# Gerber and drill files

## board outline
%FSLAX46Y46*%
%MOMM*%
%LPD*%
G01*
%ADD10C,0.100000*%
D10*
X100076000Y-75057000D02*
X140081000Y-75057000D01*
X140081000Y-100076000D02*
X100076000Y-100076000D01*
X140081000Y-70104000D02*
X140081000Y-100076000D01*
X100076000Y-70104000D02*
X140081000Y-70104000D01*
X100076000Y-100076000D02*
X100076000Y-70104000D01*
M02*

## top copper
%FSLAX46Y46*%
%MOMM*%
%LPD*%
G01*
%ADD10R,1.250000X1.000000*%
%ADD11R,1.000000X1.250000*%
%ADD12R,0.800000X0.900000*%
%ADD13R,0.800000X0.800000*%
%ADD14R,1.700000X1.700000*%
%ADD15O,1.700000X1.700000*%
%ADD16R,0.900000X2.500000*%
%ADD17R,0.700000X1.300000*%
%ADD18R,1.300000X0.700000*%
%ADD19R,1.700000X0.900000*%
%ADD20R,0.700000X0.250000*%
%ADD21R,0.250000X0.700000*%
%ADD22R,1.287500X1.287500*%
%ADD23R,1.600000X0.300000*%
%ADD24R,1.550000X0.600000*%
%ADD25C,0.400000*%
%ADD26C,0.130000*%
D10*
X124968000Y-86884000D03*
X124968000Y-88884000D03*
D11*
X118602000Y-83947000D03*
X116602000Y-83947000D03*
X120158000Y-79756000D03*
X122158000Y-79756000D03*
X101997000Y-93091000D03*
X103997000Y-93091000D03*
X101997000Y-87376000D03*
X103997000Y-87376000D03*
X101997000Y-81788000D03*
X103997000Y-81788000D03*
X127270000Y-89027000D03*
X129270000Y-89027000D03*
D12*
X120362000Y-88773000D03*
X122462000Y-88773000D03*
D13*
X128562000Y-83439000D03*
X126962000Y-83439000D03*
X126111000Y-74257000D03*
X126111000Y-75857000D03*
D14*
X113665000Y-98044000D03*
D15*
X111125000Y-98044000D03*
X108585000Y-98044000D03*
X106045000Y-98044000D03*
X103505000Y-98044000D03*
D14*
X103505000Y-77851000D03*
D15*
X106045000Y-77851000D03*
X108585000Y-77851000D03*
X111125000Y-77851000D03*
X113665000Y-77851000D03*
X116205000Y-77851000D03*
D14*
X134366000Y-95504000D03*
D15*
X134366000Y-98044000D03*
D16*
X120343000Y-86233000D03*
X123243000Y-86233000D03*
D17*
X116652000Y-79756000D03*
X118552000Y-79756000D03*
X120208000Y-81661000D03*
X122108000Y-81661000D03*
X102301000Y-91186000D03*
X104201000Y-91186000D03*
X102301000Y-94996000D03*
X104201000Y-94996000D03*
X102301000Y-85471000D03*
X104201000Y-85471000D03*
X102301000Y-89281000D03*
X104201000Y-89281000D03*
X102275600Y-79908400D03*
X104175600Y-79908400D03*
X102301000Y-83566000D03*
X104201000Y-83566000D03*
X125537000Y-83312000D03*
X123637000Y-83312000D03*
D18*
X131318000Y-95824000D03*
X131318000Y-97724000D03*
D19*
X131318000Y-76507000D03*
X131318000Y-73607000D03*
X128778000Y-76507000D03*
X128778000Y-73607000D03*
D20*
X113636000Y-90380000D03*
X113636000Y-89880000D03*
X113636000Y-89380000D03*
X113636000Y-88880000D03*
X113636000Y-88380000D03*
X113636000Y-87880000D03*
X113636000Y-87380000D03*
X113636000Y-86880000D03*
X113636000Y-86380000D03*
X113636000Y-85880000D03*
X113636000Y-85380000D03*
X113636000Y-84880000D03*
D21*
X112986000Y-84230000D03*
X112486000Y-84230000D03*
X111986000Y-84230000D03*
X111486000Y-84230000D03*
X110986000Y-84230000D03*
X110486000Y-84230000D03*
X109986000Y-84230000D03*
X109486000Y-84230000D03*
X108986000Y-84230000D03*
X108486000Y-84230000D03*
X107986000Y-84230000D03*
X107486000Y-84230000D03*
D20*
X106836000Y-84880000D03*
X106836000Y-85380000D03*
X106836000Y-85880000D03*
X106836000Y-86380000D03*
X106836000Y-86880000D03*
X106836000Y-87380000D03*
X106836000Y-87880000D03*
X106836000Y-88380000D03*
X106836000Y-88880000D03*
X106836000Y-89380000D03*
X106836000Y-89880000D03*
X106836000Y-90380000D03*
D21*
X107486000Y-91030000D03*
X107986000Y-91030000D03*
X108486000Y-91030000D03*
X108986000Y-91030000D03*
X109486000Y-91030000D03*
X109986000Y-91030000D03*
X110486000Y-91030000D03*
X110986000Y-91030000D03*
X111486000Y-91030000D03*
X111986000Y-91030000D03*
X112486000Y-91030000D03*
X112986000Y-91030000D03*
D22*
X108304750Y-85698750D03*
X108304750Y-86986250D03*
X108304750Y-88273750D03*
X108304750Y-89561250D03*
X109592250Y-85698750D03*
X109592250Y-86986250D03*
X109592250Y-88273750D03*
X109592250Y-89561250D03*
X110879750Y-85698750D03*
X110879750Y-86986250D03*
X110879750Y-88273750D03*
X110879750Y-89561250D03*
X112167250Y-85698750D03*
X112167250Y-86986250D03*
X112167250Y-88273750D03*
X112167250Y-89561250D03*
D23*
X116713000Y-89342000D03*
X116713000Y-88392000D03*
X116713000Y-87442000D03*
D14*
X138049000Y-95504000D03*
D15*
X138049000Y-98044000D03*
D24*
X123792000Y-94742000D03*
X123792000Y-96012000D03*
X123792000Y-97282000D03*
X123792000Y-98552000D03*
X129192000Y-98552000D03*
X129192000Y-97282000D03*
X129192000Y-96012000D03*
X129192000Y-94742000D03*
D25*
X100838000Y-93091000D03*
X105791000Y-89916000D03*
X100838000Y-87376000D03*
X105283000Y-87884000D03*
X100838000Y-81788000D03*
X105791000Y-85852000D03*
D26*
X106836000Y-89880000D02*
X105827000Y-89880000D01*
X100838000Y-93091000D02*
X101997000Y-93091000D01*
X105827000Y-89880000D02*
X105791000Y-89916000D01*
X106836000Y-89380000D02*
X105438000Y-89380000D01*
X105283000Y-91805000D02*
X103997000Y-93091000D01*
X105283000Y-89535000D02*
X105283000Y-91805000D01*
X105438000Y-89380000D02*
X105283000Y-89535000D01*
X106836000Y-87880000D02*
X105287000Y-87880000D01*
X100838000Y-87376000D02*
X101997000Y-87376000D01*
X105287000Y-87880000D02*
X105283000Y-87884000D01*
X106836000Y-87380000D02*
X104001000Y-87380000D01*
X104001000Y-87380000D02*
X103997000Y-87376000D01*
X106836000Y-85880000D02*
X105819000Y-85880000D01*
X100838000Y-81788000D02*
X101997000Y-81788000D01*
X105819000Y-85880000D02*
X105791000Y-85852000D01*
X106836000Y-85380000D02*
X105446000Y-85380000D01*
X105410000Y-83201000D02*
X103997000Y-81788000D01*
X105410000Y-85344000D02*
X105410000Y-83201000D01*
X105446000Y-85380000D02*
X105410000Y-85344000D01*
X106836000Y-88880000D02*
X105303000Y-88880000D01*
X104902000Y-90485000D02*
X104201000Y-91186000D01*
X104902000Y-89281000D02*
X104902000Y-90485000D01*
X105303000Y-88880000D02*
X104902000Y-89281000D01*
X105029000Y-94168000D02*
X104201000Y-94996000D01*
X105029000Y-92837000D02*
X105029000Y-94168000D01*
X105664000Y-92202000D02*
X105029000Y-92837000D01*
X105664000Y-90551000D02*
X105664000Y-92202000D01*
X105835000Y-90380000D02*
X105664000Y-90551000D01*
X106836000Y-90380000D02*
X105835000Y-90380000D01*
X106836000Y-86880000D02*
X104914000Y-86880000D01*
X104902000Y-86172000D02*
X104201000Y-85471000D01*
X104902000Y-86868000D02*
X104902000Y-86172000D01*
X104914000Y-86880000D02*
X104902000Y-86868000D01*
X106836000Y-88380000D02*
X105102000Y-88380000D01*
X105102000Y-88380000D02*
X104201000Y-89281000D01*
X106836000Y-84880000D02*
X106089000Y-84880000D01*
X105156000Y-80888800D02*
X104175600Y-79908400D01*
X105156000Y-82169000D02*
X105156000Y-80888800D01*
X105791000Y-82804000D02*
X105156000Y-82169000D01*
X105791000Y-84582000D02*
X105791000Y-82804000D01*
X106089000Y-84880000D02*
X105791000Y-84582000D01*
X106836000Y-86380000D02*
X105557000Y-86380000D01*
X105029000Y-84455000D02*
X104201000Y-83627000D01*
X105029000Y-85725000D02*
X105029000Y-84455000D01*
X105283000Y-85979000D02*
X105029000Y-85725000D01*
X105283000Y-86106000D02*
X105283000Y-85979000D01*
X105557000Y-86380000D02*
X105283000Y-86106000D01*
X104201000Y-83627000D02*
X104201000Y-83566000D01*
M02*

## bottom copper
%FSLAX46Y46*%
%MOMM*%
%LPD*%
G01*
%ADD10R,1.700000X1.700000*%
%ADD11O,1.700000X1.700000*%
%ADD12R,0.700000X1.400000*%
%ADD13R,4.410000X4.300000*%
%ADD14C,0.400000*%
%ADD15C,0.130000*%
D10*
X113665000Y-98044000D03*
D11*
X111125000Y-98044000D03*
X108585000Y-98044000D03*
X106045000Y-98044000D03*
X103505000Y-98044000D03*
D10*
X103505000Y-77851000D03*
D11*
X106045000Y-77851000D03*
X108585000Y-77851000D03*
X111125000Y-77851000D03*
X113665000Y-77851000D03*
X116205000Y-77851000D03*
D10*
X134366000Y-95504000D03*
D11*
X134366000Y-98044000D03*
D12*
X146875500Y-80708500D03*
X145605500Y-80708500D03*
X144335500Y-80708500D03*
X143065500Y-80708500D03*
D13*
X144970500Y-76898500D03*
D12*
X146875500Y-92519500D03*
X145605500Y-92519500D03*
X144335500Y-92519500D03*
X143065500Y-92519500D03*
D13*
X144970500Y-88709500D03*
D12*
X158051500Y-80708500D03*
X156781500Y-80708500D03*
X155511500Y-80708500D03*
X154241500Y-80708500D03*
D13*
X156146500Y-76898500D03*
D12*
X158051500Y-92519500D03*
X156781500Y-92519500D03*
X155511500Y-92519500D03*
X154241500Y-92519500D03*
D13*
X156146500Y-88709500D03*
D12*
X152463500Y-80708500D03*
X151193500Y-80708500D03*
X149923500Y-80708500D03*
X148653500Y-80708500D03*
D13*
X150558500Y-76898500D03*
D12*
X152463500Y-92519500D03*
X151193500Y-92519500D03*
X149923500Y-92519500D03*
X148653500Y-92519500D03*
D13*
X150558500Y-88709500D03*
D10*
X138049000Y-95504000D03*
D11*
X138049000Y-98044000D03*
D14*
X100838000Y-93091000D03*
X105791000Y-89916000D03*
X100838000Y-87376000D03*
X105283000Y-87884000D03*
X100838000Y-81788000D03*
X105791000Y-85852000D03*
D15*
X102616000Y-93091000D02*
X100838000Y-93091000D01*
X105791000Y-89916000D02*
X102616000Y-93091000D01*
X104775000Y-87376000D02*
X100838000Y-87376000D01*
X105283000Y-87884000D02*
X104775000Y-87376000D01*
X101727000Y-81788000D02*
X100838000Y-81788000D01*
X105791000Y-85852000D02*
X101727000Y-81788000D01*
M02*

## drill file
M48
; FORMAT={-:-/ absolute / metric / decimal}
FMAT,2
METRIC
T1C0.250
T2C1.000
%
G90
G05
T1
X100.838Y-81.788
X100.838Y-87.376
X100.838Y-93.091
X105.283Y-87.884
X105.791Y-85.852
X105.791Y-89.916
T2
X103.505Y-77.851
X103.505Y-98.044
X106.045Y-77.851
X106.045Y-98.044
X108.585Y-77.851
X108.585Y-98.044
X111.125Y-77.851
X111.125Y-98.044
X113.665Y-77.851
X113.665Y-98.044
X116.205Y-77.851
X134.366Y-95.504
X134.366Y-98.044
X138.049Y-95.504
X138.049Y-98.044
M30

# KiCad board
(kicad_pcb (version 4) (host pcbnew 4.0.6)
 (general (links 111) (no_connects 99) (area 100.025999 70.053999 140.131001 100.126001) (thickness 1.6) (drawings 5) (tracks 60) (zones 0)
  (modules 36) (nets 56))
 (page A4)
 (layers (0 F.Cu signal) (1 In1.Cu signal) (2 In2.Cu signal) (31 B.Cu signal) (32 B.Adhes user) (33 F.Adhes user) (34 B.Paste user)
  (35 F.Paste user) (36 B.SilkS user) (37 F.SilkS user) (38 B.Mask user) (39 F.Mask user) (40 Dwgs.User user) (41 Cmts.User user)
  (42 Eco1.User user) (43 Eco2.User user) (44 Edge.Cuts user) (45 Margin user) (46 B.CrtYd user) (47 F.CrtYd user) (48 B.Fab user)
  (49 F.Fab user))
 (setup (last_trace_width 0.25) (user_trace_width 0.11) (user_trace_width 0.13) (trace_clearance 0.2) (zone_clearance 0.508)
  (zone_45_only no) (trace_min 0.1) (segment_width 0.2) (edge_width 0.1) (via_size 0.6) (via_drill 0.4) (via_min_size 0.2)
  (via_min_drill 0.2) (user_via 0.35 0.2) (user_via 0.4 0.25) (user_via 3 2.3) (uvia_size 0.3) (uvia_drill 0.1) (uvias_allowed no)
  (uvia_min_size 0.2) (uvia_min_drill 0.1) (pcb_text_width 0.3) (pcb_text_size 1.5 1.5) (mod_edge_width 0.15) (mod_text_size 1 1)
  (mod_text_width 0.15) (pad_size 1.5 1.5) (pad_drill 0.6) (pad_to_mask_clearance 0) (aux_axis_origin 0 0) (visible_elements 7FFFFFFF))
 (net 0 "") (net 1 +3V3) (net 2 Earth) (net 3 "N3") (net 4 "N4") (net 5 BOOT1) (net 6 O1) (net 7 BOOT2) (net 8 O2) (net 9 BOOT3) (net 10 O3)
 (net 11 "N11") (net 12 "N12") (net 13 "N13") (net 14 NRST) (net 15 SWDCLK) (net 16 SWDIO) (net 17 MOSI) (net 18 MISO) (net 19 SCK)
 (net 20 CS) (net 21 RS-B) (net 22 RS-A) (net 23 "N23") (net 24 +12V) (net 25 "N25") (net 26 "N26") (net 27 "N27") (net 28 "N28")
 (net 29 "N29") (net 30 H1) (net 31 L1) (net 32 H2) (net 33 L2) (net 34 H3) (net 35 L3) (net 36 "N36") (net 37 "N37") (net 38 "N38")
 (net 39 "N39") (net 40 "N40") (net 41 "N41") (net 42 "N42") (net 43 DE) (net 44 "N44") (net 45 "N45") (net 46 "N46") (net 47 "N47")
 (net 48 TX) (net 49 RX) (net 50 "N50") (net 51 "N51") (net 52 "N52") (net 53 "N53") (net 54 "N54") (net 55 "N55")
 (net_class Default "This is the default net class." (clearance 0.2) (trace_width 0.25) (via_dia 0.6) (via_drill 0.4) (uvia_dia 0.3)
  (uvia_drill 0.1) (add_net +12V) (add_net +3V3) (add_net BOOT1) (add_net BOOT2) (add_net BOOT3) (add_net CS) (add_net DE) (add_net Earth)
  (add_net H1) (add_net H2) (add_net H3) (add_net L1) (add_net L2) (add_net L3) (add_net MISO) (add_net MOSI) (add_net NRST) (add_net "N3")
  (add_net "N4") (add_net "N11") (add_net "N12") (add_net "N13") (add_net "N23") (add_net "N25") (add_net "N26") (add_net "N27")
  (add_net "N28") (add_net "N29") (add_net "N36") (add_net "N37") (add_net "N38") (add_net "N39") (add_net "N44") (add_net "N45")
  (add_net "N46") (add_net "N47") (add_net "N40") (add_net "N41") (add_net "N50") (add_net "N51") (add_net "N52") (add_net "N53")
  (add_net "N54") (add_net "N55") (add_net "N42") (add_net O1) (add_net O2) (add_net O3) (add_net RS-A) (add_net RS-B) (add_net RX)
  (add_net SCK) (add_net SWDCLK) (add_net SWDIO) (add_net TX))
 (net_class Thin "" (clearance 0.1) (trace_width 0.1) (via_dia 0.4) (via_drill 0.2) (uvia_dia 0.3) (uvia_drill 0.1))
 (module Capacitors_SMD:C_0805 (layer F.Cu) (at 124.968 87.884 270)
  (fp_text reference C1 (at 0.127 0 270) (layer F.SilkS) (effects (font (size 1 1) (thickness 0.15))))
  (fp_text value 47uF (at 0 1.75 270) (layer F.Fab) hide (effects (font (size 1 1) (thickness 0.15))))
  (pad 1 smd rect (at -1 0 270) (size 1 1.25) (layers F.Cu F.Paste F.Mask) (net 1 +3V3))
  (pad 2 smd rect (at 1 0 270) (size 1 1.25) (layers F.Cu F.Paste F.Mask) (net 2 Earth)))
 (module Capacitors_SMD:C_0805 (layer F.Cu) (at 117.602 83.947 180)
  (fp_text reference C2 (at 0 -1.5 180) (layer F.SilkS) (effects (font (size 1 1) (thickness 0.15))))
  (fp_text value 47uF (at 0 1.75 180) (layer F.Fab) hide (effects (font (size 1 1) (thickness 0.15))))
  (pad 1 smd rect (at -1 0 180) (size 1 1.25) (layers F.Cu F.Paste F.Mask) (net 2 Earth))
  (pad 2 smd rect (at 1 0 180) (size 1 1.25) (layers F.Cu F.Paste F.Mask) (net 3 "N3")))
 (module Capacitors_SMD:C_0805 (layer F.Cu) (at 121.158 79.756)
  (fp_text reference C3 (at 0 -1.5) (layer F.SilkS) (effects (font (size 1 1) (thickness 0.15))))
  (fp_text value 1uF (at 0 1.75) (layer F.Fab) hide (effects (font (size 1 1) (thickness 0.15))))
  (pad 1 smd rect (at -1 0) (size 1 1.25) (layers F.Cu F.Paste F.Mask) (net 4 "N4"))
  (pad 2 smd rect (at 1 0) (size 1 1.25) (layers F.Cu F.Paste F.Mask) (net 2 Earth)))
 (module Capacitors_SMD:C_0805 (layer F.Cu) (at 102.997 93.091)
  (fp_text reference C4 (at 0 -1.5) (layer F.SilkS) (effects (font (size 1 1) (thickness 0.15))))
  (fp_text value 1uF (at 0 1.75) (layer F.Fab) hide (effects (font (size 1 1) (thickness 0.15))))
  (pad 1 smd rect (at -1 0) (size 1 1.25) (layers F.Cu F.Paste F.Mask) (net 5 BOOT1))
  (pad 2 smd rect (at 1 0) (size 1 1.25) (layers F.Cu F.Paste F.Mask) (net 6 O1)))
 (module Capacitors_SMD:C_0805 (layer F.Cu) (at 102.997 87.376)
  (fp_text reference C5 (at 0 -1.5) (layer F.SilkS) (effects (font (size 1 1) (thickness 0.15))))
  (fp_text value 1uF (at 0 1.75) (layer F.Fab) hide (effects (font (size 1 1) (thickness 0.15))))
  (pad 1 smd rect (at -1 0) (size 1 1.25) (layers F.Cu F.Paste F.Mask) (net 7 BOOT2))
  (pad 2 smd rect (at 1 0) (size 1 1.25) (layers F.Cu F.Paste F.Mask) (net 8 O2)))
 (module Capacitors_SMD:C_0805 (layer F.Cu) (at 102.997 81.788)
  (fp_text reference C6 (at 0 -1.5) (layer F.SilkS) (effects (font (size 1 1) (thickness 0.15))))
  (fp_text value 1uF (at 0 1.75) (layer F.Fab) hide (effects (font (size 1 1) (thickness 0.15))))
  (pad 1 smd rect (at -1 0) (size 1 1.25) (layers F.Cu F.Paste F.Mask) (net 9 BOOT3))
  (pad 2 smd rect (at 1 0) (size 1 1.25) (layers F.Cu F.Paste F.Mask) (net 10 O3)))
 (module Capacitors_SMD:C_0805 (layer F.Cu) (at 128.27 89.027)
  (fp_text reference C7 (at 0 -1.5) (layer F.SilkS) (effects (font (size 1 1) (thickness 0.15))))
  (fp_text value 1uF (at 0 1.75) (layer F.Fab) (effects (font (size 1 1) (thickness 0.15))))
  (pad 1 smd rect (at -1 0) (size 1 1.25) (layers F.Cu F.Paste F.Mask) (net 2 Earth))
  (pad 2 smd rect (at 1 0) (size 1 1.25) (layers F.Cu F.Paste F.Mask) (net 1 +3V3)))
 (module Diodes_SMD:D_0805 (layer F.Cu) (at 121.412 88.773)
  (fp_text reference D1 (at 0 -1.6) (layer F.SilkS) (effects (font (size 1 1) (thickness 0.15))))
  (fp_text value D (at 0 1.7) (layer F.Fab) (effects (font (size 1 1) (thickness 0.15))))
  (pad 1 smd rect (at -1.05 0) (size 0.8 0.9) (layers F.Cu F.Paste F.Mask) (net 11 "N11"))
  (pad 2 smd rect (at 1.05 0) (size 0.8 0.9) (layers F.Cu F.Paste F.Mask) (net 2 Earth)))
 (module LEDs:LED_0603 (layer F.Cu) (at 127.762 83.439)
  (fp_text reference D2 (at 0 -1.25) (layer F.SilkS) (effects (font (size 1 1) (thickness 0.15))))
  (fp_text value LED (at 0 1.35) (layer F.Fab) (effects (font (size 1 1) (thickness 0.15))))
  (pad 2 smd rect (at 0.8 0 180) (size 0.8 0.8) (layers F.Cu F.Paste F.Mask) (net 1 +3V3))
  (pad 1 smd rect (at -0.8 0 180) (size 0.8 0.8) (layers F.Cu F.Paste F.Mask) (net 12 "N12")))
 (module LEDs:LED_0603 (layer F.Cu) (at 126.111 75.057 90)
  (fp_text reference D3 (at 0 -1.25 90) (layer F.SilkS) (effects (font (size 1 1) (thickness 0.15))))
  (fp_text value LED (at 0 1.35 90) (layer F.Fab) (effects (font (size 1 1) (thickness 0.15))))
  (pad 2 smd rect (at 0.8 0 270) (size 0.8 0.8) (layers F.Cu F.Paste F.Mask) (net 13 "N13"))
  (pad 1 smd rect (at -0.8 0 270) (size 0.8 0.8) (layers F.Cu F.Paste F.Mask) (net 2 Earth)))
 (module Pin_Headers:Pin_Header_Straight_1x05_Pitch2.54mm (layer F.Cu) (at 113.665 98.044 270)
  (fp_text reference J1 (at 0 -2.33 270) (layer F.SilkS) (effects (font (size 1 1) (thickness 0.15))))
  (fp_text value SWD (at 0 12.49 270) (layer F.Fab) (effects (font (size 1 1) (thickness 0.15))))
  (pad 1 thru_hole rect (at 0 0 270) (size 1.7 1.7) (drill 1) (layers *.Cu *.Mask) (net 1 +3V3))
  (pad 2 thru_hole oval (at 0 2.54 270) (size 1.7 1.7) (drill 1) (layers *.Cu *.Mask) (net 2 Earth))
  (pad 3 thru_hole oval (at 0 5.08 270) (size 1.7 1.7) (drill 1) (layers *.Cu *.Mask) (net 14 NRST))
  (pad 4 thru_hole oval (at 0 7.62 270) (size 1.7 1.7) (drill 1) (layers *.Cu *.Mask) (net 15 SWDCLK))
  (pad 5 thru_hole oval (at 0 10.16 270) (size 1.7 1.7) (drill 1) (layers *.Cu *.Mask) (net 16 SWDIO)))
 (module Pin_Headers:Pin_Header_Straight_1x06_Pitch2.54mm (layer F.Cu) (at 103.505 77.851 90)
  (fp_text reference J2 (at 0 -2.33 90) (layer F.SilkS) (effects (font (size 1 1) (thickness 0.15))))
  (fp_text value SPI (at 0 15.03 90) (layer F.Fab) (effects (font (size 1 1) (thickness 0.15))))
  (pad 1 thru_hole rect (at 0 0 90) (size 1.7 1.7) (drill 1) (layers *.Cu *.Mask) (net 1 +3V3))
  (pad 2 thru_hole oval (at 0 2.54 90) (size 1.7 1.7) (drill 1) (layers *.Cu *.Mask) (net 2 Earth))
  (pad 3 thru_hole oval (at 0 5.08 90) (size 1.7 1.7) (drill 1) (layers *.Cu *.Mask) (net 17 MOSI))
  (pad 4 thru_hole oval (at 0 7.62 90) (size 1.7 1.7) (drill 1) (layers *.Cu *.Mask) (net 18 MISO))
  (pad 5 thru_hole oval (at 0 10.16 90) (size 1.7 1.7) (drill 1) (layers *.Cu *.Mask) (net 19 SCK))
  (pad 6 thru_hole oval (at 0 12.7 90) (size 1.7 1.7) (drill 1) (layers *.Cu *.Mask) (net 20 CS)))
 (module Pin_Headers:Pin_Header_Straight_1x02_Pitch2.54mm (layer F.Cu) (at 134.366 95.504)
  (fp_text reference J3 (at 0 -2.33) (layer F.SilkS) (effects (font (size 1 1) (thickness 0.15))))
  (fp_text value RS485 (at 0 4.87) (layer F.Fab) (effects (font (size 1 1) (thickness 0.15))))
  (pad 1 thru_hole rect (at 0 0) (size 1.7 1.7) (drill 1) (layers *.Cu *.Mask) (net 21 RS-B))
  (pad 2 thru_hole oval (at 0 2.54) (size 1.7 1.7) (drill 1) (layers *.Cu *.Mask) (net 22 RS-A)))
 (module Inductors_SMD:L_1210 (layer F.Cu) (at 121.793 86.233)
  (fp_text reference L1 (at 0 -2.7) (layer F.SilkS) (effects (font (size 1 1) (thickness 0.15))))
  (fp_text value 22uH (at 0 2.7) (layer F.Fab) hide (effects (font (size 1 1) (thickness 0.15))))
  (pad 1 smd rect (at -1.45 0) (size 0.9 2.5) (layers F.Cu F.Paste F.Mask) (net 11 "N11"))
  (pad 2 smd rect (at 1.45 0) (size 0.9 2.5) (layers F.Cu F.Paste F.Mask) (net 1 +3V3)))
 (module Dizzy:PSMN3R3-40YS (layer B.Cu) (at 144.9705 78.1685 180)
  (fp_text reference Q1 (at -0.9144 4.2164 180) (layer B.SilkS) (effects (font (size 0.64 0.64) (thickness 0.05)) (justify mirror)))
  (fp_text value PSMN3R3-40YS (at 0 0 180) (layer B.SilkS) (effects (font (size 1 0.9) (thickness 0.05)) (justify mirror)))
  (pad 1 smd rect (at -1.905 -2.54 270) (size 1.4 0.7) (layers B.Cu B.Paste B.Mask) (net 6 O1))
  (pad 2 smd rect (at -0.635 -2.54 270) (size 1.4 0.7) (layers B.Cu B.Paste B.Mask) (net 6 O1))
  (pad 3 smd rect (at 0.635 -2.54 270) (size 1.4 0.7) (layers B.Cu B.Paste B.Mask) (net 6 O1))
  (pad 4 smd rect (at 1.905 -2.54 270) (size 1.4 0.7) (layers B.Cu B.Paste B.Mask) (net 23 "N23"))
  (pad 5678 smd rect (at 0 1.27 270) (size 4.3 4.41) (layers B.Cu B.Paste B.Mask) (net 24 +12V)))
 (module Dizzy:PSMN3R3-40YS (layer B.Cu) (at 144.9705 89.9795 180)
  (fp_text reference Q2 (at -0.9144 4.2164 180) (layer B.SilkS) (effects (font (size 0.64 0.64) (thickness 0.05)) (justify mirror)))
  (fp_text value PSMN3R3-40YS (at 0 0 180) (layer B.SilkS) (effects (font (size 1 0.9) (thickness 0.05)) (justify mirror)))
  (pad 1 smd rect (at -1.905 -2.54 270) (size 1.4 0.7) (layers B.Cu B.Paste B.Mask) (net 2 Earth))
  (pad 2 smd rect (at -0.635 -2.54 270) (size 1.4 0.7) (layers B.Cu B.Paste B.Mask) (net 2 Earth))
  (pad 3 smd rect (at 0.635 -2.54 270) (size 1.4 0.7) (layers B.Cu B.Paste B.Mask) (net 2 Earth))
  (pad 4 smd rect (at 1.905 -2.54 270) (size 1.4 0.7) (layers B.Cu B.Paste B.Mask) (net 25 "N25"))
  (pad 5678 smd rect (at 0 1.27 270) (size 4.3 4.41) (layers B.Cu B.Paste B.Mask) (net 6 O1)))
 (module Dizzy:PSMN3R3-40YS (layer B.Cu) (at 156.1465 78.1685 180)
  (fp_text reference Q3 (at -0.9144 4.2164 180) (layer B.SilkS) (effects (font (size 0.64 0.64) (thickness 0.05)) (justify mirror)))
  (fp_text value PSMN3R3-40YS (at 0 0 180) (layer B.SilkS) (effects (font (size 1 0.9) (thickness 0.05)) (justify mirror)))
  (pad 1 smd rect (at -1.905 -2.54 270) (size 1.4 0.7) (layers B.Cu B.Paste B.Mask) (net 8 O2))
  (pad 2 smd rect (at -0.635 -2.54 270) (size 1.4 0.7) (layers B.Cu B.Paste B.Mask) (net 8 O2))
  (pad 3 smd rect (at 0.635 -2.54 270) (size 1.4 0.7) (layers B.Cu B.Paste B.Mask) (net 8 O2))
  (pad 4 smd rect (at 1.905 -2.54 270) (size 1.4 0.7) (layers B.Cu B.Paste B.Mask) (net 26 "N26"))
  (pad 5678 smd rect (at 0 1.27 270) (size 4.3 4.41) (layers B.Cu B.Paste B.Mask) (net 24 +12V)))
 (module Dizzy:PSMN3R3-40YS (layer B.Cu) (at 156.1465 89.9795 180)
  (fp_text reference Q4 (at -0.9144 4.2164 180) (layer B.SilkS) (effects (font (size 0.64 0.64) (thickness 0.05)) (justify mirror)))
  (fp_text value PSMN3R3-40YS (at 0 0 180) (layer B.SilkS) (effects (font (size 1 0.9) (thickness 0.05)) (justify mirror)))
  (pad 1 smd rect (at -1.905 -2.54 270) (size 1.4 0.7) (layers B.Cu B.Paste B.Mask) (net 2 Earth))
  (pad 2 smd rect (at -0.635 -2.54 270) (size 1.4 0.7) (layers B.Cu B.Paste B.Mask) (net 2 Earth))
  (pad 3 smd rect (at 0.635 -2.54 270) (size 1.4 0.7) (layers B.Cu B.Paste B.Mask) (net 2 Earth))
  (pad 4 smd rect (at 1.905 -2.54 270) (size 1.4 0.7) (layers B.Cu B.Paste B.Mask) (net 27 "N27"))
  (pad 5678 smd rect (at 0 1.27 270) (size 4.3 4.41) (layers B.Cu B.Paste B.Mask) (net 8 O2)))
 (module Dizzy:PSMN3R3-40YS (layer B.Cu) (at 150.5585 78.1685 180)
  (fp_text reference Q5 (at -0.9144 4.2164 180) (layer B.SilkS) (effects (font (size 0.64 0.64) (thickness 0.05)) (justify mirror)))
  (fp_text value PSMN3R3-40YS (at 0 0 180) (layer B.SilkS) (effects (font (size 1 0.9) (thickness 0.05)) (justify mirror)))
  (pad 1 smd rect (at -1.905 -2.54 270) (size 1.4 0.7) (layers B.Cu B.Paste B.Mask) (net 10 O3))
  (pad 2 smd rect (at -0.635 -2.54 270) (size 1.4 0.7) (layers B.Cu B.Paste B.Mask) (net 10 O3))
  (pad 3 smd rect (at 0.635 -2.54 270) (size 1.4 0.7) (layers B.Cu B.Paste B.Mask) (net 10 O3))
  (pad 4 smd rect (at 1.905 -2.54 270) (size 1.4 0.7) (layers B.Cu B.Paste B.Mask) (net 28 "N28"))
  (pad 5678 smd rect (at 0 1.27 270) (size 4.3 4.41) (layers B.Cu B.Paste B.Mask) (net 24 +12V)))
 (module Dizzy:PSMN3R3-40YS (layer B.Cu) (at 150.5585 89.9795 180)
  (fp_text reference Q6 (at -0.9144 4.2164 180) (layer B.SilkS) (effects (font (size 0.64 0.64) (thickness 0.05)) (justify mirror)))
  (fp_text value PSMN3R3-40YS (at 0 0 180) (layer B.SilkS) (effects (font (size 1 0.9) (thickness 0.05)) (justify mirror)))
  (pad 1 smd rect (at -1.905 -2.54 270) (size 1.4 0.7) (layers B.Cu B.Paste B.Mask) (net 2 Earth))
  (pad 2 smd rect (at -0.635 -2.54 270) (size 1.4 0.7) (layers B.Cu B.Paste B.Mask) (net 2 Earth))
  (pad 3 smd rect (at 0.635 -2.54 270) (size 1.4 0.7) (layers B.Cu B.Paste B.Mask) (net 2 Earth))
  (pad 4 smd rect (at 1.905 -2.54 270) (size 1.4 0.7) (layers B.Cu B.Paste B.Mask) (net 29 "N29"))
  (pad 5678 smd rect (at 0 1.27 270) (size 4.3 4.41) (layers B.Cu B.Paste B.Mask) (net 10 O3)))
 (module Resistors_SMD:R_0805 (layer F.Cu) (at 117.602 79.756)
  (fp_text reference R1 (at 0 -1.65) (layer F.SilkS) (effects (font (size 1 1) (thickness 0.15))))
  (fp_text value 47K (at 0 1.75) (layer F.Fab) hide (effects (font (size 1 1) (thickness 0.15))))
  (pad 1 smd rect (at -0.95 0) (size 0.7 1.3) (layers F.Cu F.Paste F.Mask) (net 24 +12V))
  (pad 2 smd rect (at 0.95 0) (size 0.7 1.3) (layers F.Cu F.Paste F.Mask) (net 4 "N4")))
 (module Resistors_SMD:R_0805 (layer F.Cu) (at 121.158 81.661)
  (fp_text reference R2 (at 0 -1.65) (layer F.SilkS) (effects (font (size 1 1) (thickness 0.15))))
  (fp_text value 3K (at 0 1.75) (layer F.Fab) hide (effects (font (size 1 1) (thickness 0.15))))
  (pad 1 smd rect (at -0.95 0) (size 0.7 1.3) (layers F.Cu F.Paste F.Mask) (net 4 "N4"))
  (pad 2 smd rect (at 0.95 0) (size 0.7 1.3) (layers F.Cu F.Paste F.Mask) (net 2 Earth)))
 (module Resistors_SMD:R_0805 (layer F.Cu) (at 103.251 91.186)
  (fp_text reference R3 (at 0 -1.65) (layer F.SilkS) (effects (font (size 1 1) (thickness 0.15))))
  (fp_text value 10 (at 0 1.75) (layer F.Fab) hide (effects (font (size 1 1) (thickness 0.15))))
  (pad 1 smd rect (at -0.95 0) (size 0.7 1.3) (layers F.Cu F.Paste F.Mask) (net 23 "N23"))
  (pad 2 smd rect (at 0.95 0) (size 0.7 1.3) (layers F.Cu F.Paste F.Mask) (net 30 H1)))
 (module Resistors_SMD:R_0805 (layer F.Cu) (at 103.251 94.996)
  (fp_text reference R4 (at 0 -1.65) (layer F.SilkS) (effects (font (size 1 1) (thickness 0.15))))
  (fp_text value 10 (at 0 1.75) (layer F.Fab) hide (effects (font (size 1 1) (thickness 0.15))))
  (pad 1 smd rect (at -0.95 0) (size 0.7 1.3) (layers F.Cu F.Paste F.Mask) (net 25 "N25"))
  (pad 2 smd rect (at 0.95 0) (size 0.7 1.3) (layers F.Cu F.Paste F.Mask) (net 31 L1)))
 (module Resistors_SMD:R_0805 (layer F.Cu) (at 103.251 85.471)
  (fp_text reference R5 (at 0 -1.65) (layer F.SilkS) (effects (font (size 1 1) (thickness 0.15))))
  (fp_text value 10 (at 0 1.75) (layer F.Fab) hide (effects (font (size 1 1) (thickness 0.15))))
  (pad 1 smd rect (at -0.95 0) (size 0.7 1.3) (layers F.Cu F.Paste F.Mask) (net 26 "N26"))
  (pad 2 smd rect (at 0.95 0) (size 0.7 1.3) (layers F.Cu F.Paste F.Mask) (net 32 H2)))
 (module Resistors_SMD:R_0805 (layer F.Cu) (at 103.251 89.281)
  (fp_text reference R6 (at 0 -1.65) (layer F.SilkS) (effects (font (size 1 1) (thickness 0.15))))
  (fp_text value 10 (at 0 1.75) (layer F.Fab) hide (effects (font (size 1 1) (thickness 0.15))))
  (pad 1 smd rect (at -0.95 0) (size 0.7 1.3) (layers F.Cu F.Paste F.Mask) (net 27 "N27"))
  (pad 2 smd rect (at 0.95 0) (size 0.7 1.3) (layers F.Cu F.Paste F.Mask) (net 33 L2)))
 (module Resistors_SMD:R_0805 (layer F.Cu) (at 103.2256 79.9084)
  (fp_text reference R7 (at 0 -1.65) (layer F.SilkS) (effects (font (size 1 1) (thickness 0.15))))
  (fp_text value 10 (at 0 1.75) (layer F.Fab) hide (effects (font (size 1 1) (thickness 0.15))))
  (pad 1 smd rect (at -0.95 0) (size 0.7 1.3) (layers F.Cu F.Paste F.Mask) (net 28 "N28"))
  (pad 2 smd rect (at 0.95 0) (size 0.7 1.3) (layers F.Cu F.Paste F.Mask) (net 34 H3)))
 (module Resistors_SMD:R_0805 (layer F.Cu) (at 103.251 83.566)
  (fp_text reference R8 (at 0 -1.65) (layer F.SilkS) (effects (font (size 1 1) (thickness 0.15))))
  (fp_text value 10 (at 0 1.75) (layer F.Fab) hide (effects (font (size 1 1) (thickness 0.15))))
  (pad 1 smd rect (at -0.95 0) (size 0.7 1.3) (layers F.Cu F.Paste F.Mask) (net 29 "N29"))
  (pad 2 smd rect (at 0.95 0) (size 0.7 1.3) (layers F.Cu F.Paste F.Mask) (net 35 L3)))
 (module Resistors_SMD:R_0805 (layer F.Cu) (at 124.587 83.312 180)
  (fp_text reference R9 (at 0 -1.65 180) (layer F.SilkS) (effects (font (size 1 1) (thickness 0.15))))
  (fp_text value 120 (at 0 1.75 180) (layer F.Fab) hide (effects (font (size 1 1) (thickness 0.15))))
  (pad 1 smd rect (at -0.95 0 180) (size 0.7 1.3) (layers F.Cu F.Paste F.Mask) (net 12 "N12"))
  (pad 2 smd rect (at 0.95 0 180) (size 0.7 1.3) (layers F.Cu F.Paste F.Mask) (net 2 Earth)))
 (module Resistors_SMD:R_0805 (layer F.Cu) (at 131.318 96.774 270)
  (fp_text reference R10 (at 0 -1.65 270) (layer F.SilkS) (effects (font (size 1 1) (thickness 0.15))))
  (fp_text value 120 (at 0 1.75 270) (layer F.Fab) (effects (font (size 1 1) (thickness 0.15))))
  (pad 1 smd rect (at -0.95 0 270) (size 0.7 1.3) (layers F.Cu F.Paste F.Mask) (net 21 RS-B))
  (pad 2 smd rect (at 0.95 0 270) (size 0.7 1.3) (layers F.Cu F.Paste F.Mask) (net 22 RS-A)))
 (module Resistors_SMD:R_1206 (layer F.Cu) (at 131.318 75.057 90)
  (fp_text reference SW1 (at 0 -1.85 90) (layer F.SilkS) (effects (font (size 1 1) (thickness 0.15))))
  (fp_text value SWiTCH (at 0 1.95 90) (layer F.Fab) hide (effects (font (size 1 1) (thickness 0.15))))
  (pad 1 smd rect (at -1.45 0 90) (size 0.9 1.7) (layers F.Cu F.Paste F.Mask) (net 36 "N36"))
  (pad 2 smd rect (at 1.45 0 90) (size 0.9 1.7) (layers F.Cu F.Paste F.Mask) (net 1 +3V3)))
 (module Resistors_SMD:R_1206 (layer F.Cu) (at 128.778 75.057 90)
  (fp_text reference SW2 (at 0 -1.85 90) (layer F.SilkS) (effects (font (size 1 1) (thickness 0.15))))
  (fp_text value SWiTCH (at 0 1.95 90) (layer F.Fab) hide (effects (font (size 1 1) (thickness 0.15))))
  (pad 1 smd rect (at -1.45 0 90) (size 0.9 1.7) (layers F.Cu F.Paste F.Mask) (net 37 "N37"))
  (pad 2 smd rect (at 1.45 0 90) (size 0.9 1.7) (layers F.Cu F.Paste F.Mask) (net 1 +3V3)))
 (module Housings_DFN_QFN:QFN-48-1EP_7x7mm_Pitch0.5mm (layer F.Cu) (at 110.236 87.63 180)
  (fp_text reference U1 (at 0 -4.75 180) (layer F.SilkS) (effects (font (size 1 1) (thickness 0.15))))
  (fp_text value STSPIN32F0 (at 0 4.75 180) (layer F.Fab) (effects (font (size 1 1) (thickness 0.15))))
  (pad 1 smd rect (at -3.4 -2.75 180) (size 0.7 0.25) (layers F.Cu F.Paste F.Mask) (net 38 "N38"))
  (pad 2 smd rect (at -3.4 -2.25 180) (size 0.7 0.25) (layers F.Cu F.Paste F.Mask) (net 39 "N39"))
  (pad 3 smd rect (at -3.4 -1.75 180) (size 0.7 0.25) (layers F.Cu F.Paste F.Mask) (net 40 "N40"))
  (pad 4 smd rect (at -3.4 -1.25 180) (size 0.7 0.25) (layers F.Cu F.Paste F.Mask) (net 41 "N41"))
  (pad 5 smd rect (at -3.4 -0.75 180) (size 0.7 0.25) (layers F.Cu F.Paste F.Mask) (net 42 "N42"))
  (pad 6 smd rect (at -3.4 -0.25 180) (size 0.7 0.25) (layers F.Cu F.Paste F.Mask) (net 3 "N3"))
  (pad 7 smd rect (at -3.4 0.25 180) (size 0.7 0.25) (layers F.Cu F.Paste F.Mask) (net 14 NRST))
  (pad 8 smd rect (at -3.4 0.75 180) (size 0.7 0.25) (layers F.Cu F.Paste F.Mask) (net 24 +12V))
  (pad 9 smd rect (at -3.4 1.25 180) (size 0.7 0.25) (layers F.Cu F.Paste F.Mask) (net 11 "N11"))
  (pad 10 smd rect (at -3.4 1.75 180) (size 0.7 0.25) (layers F.Cu F.Paste F.Mask) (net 1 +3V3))
  (pad 11 smd rect (at -3.4 2.25 180) (size 0.7 0.25) (layers F.Cu F.Paste F.Mask) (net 4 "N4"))
  (pad 12 smd rect (at -3.4 2.75 180) (size 0.7 0.25) (layers F.Cu F.Paste F.Mask) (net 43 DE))
  (pad 13 smd rect (at -2.75 3.4 270) (size 0.7 0.25) (layers F.Cu F.Paste F.Mask) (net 36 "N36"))
  (pad 14 smd rect (at -2.25 3.4 270) (size 0.7 0.25) (layers F.Cu F.Paste F.Mask) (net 37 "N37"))
  (pad 15 smd rect (at -1.75 3.4 270) (size 0.7 0.25) (layers F.Cu F.Paste F.Mask) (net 20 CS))
  (pad 16 smd rect (at -1.25 3.4 270) (size 0.7 0.25) (layers F.Cu F.Paste F.Mask) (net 19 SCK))
  (pad 17 smd rect (at -0.75 3.4 270) (size 0.7 0.25) (layers F.Cu F.Paste F.Mask) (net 18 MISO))
  (pad 18 smd rect (at -0.25 3.4 270) (size 0.7 0.25) (layers F.Cu F.Paste F.Mask) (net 17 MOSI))
  (pad 19 smd rect (at 0.25 3.4 270) (size 0.7 0.25) (layers F.Cu F.Paste F.Mask) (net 13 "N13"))
  (pad 20 smd rect (at 0.75 3.4 270) (size 0.7 0.25) (layers F.Cu F.Paste F.Mask) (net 2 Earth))
  (pad 21 smd rect (at 1.25 3.4 270) (size 0.7 0.25) (layers F.Cu F.Paste F.Mask) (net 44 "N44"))
  (pad 22 smd rect (at 1.75 3.4 270) (size 0.7 0.25) (layers F.Cu F.Paste F.Mask) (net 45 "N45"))
  (pad 23 smd rect (at 2.25 3.4 270) (size 0.7 0.25) (layers F.Cu F.Paste F.Mask) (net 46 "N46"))
  (pad 24 smd rect (at 2.75 3.4 270) (size 0.7 0.25) (layers F.Cu F.Paste F.Mask) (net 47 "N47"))
  (pad 25 smd rect (at 3.4 2.75 180) (size 0.7 0.25) (layers F.Cu F.Paste F.Mask) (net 34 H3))
  (pad 26 smd rect (at 3.4 2.25 180) (size 0.7 0.25) (layers F.Cu F.Paste F.Mask) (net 10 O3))
  (pad 27 smd rect (at 3.4 1.75 180) (size 0.7 0.25) (layers F.Cu F.Paste F.Mask) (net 9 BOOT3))
  (pad 28 smd rect (at 3.4 1.25 180) (size 0.7 0.25) (layers F.Cu F.Paste F.Mask) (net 35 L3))
  (pad 29 smd rect (at 3.4 0.75 180) (size 0.7 0.25) (layers F.Cu F.Paste F.Mask) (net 32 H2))
  (pad 30 smd rect (at 3.4 0.25 180) (size 0.7 0.25) (layers F.Cu F.Paste F.Mask) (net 8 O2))
  (pad 31 smd rect (at 3.4 -0.25 180) (size 0.7 0.25) (layers F.Cu F.Paste F.Mask) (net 7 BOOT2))
  (pad 32 smd rect (at 3.4 -0.75 180) (size 0.7 0.25) (layers F.Cu F.Paste F.Mask) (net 33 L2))
  (pad 33 smd rect (at 3.4 -1.25 180) (size 0.7 0.25) (layers F.Cu F.Paste F.Mask) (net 30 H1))
  (pad 34 smd rect (at 3.4 -1.75 180) (size 0.7 0.25) (layers F.Cu F.Paste F.Mask) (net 6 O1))
  (pad 35 smd rect (at 3.4 -2.25 180) (size 0.7 0.25) (layers F.Cu F.Paste F.Mask) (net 5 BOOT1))
  (pad 36 smd rect (at 3.4 -2.75 180) (size 0.7 0.25) (layers F.Cu F.Paste F.Mask) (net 31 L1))
  (pad 37 smd rect (at 2.75 -3.4 270) (size 0.7 0.25) (layers F.Cu F.Paste F.Mask) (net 16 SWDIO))
  (pad 38 smd rect (at 2.25 -3.4 270) (size 0.7 0.25) (layers F.Cu F.Paste F.Mask) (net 15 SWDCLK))
  (pad 39 smd rect (at 1.75 -3.4 270) (size 0.7 0.25) (layers F.Cu F.Paste F.Mask) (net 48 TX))
  (pad 40 smd rect (at 1.25 -3.4 270) (size 0.7 0.25) (layers F.Cu F.Paste F.Mask) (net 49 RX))
  (pad 41 smd rect (at 0.75 -3.4 270) (size 0.7 0.25) (layers F.Cu F.Paste F.Mask) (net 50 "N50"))
  (pad 42 smd rect (at 0.25 -3.4 270) (size 0.7 0.25) (layers F.Cu F.Paste F.Mask) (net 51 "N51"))
  (pad 43 smd rect (at -0.25 -3.4 270) (size 0.7 0.25) (layers F.Cu F.Paste F.Mask) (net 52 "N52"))
  (pad 44 smd rect (at -0.75 -3.4 270) (size 0.7 0.25) (layers F.Cu F.Paste F.Mask) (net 2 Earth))
  (pad 45 smd rect (at -1.25 -3.4 270) (size 0.7 0.25) (layers F.Cu F.Paste F.Mask) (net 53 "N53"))
  (pad 46 smd rect (at -1.75 -3.4 270) (size 0.7 0.25) (layers F.Cu F.Paste F.Mask) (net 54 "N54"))
  (pad 47 smd rect (at -2.25 -3.4 270) (size 0.7 0.25) (layers F.Cu F.Paste F.Mask) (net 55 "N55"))
  (pad 48 smd rect (at -2.75 -3.4 270) (size 0.7 0.25) (layers F.Cu F.Paste F.Mask) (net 1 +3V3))
  (pad 49 smd rect (at 1.93125 1.93125 180) (size 1.2875 1.2875) (layers F.Cu F.Paste F.Mask) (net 2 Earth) (solder_paste_margin_ratio -0.2))
  (pad 49 smd rect (at 1.93125 0.64375 180) (size 1.2875 1.2875) (layers F.Cu F.Paste F.Mask) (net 2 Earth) (solder_paste_margin_ratio -0.2))
  (pad 49 smd rect (at 1.93125 -0.64375 180) (size 1.2875 1.2875) (layers F.Cu F.Paste F.Mask) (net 2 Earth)
   (solder_paste_margin_ratio -0.2))
  (pad 49 smd rect (at 1.93125 -1.93125 180) (size 1.2875 1.2875) (layers F.Cu F.Paste F.Mask) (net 2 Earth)
   (solder_paste_margin_ratio -0.2))
  (pad 49 smd rect (at 0.64375 1.93125 180) (size 1.2875 1.2875) (layers F.Cu F.Paste F.Mask) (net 2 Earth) (solder_paste_margin_ratio -0.2))
  (pad 49 smd rect (at 0.64375 0.64375 180) (size 1.2875 1.2875) (layers F.Cu F.Paste F.Mask) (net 2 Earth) (solder_paste_margin_ratio -0.2))
  (pad 49 smd rect (at 0.64375 -0.64375 180) (size 1.2875 1.2875) (layers F.Cu F.Paste F.Mask) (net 2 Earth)
   (solder_paste_margin_ratio -0.2))
  (pad 49 smd rect (at 0.64375 -1.93125 180) (size 1.2875 1.2875) (layers F.Cu F.Paste F.Mask) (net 2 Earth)
   (solder_paste_margin_ratio -0.2))
  (pad 49 smd rect (at -0.64375 1.93125 180) (size 1.2875 1.2875) (layers F.Cu F.Paste F.Mask) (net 2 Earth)
   (solder_paste_margin_ratio -0.2))
  (pad 49 smd rect (at -0.64375 0.64375 180) (size 1.2875 1.2875) (layers F.Cu F.Paste F.Mask) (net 2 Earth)
   (solder_paste_margin_ratio -0.2))
  (pad 49 smd rect (at -0.64375 -0.64375 180) (size 1.2875 1.2875) (layers F.Cu F.Paste F.Mask) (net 2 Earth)
   (solder_paste_margin_ratio -0.2))
  (pad 49 smd rect (at -0.64375 -1.93125 180) (size 1.2875 1.2875) (layers F.Cu F.Paste F.Mask) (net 2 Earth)
   (solder_paste_margin_ratio -0.2))
  (pad 49 smd rect (at -1.93125 1.93125 180) (size 1.2875 1.2875) (layers F.Cu F.Paste F.Mask) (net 2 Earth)
   (solder_paste_margin_ratio -0.2))
  (pad 49 smd rect (at -1.93125 0.64375 180) (size 1.2875 1.2875) (layers F.Cu F.Paste F.Mask) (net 2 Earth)
   (solder_paste_margin_ratio -0.2))
  (pad 49 smd rect (at -1.93125 -0.64375 180) (size 1.2875 1.2875) (layers F.Cu F.Paste F.Mask) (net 2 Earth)
   (solder_paste_margin_ratio -0.2))
  (pad 49 smd rect (at -1.93125 -1.93125 180) (size 1.2875 1.2875) (layers F.Cu F.Paste F.Mask) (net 2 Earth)
   (solder_paste_margin_ratio -0.2)))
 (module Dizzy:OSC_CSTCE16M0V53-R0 (layer F.Cu) (at 116.713 88.392 90)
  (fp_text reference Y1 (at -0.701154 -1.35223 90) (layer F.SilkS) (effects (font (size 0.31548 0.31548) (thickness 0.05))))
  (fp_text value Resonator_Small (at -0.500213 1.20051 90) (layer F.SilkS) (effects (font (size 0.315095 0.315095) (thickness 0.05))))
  (pad 1 smd rect (at -0.95 0 90) (size 0.3 1.6) (layers F.Cu F.Paste F.Mask) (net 41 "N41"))
  (pad 2 smd rect (at 0 0 90) (size 0.3 1.6) (layers F.Cu F.Paste F.Mask) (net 2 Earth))
  (pad 3 smd rect (at 0.95 0 90) (size 0.3 1.6) (layers F.Cu F.Paste F.Mask) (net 42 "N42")))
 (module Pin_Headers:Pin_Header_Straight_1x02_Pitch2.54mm (layer F.Cu) (at 138.049 95.504)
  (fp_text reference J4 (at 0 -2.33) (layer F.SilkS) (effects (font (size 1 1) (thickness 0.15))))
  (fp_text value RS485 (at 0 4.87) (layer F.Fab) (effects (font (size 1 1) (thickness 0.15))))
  (pad 1 thru_hole rect (at 0 0) (size 1.7 1.7) (drill 1) (layers *.Cu *.Mask) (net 21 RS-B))
  (pad 2 thru_hole oval (at 0 2.54) (size 1.7 1.7) (drill 1) (layers *.Cu *.Mask) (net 22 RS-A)))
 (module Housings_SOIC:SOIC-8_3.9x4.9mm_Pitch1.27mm (layer F.Cu) (at 126.492 96.647)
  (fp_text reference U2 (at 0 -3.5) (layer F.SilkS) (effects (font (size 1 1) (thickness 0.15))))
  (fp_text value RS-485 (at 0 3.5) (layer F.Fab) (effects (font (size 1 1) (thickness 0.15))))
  (pad 1 smd rect (at -2.7 -1.905) (size 1.55 0.6) (layers F.Cu F.Paste F.Mask) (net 49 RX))
  (pad 2 smd rect (at -2.7 -0.635) (size 1.55 0.6) (layers F.Cu F.Paste F.Mask) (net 2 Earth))
  (pad 3 smd rect (at -2.7 0.635) (size 1.55 0.6) (layers F.Cu F.Paste F.Mask) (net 43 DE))
  (pad 4 smd rect (at -2.7 1.905) (size 1.55 0.6) (layers F.Cu F.Paste F.Mask) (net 48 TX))
  (pad 5 smd rect (at 2.7 1.905) (size 1.55 0.6) (layers F.Cu F.Paste F.Mask) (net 2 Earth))
  (pad 6 smd rect (at 2.7 0.635) (size 1.55 0.6) (layers F.Cu F.Paste F.Mask) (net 22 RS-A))
  (pad 7 smd rect (at 2.7 -0.635) (size 1.55 0.6) (layers F.Cu F.Paste F.Mask) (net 21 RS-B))
  (pad 8 smd rect (at 2.7 -1.905) (size 1.55 0.6) (layers F.Cu F.Paste F.Mask) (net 1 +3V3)))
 (gr_line (start 100.076 75.057) (end 140.081 75.057) (angle 90) (layer Edge.Cuts) (width 0.1))
 (gr_line (start 140.081 100.076) (end 100.076 100.076) (angle 90) (layer Edge.Cuts) (width 0.1))
 (gr_line (start 140.081 70.104) (end 140.081 100.076) (angle 90) (layer Edge.Cuts) (width 0.1))
 (gr_line (start 100.076 70.104) (end 140.081 70.104) (angle 90) (layer Edge.Cuts) (width 0.1))
 (gr_line (start 100.076 100.076) (end 100.076 70.104) (angle 90) (layer Edge.Cuts) (width 0.1))
 (segment (start 106.836 89.88) (end 105.827 89.88) (width 0.13) (layer F.Cu) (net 5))
 (segment (start 100.838 93.091) (end 101.997 93.091) (width 0.13) (layer F.Cu) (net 5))
 (via (at 100.838 93.091) (size 0.4) (drill 0.25) (layers F.Cu B.Cu) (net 5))
 (segment (start 102.616 93.091) (end 100.838 93.091) (width 0.13) (layer B.Cu) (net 5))
 (segment (start 105.791 89.916) (end 102.616 93.091) (width 0.13) (layer B.Cu) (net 5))
 (via (at 105.791 89.916) (size 0.4) (drill 0.25) (layers F.Cu B.Cu) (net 5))
 (segment (start 105.827 89.88) (end 105.791 89.916) (width 0.13) (layer F.Cu) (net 5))
 (segment (start 106.836 89.38) (end 105.438 89.38) (width 0.13) (layer F.Cu) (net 6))
 (segment (start 105.283 91.805) (end 103.997 93.091) (width 0.13) (layer F.Cu) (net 6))
 (segment (start 105.283 89.535) (end 105.283 91.805) (width 0.13) (layer F.Cu) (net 6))
 (segment (start 105.438 89.38) (end 105.283 89.535) (width 0.13) (layer F.Cu) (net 6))
 (segment (start 106.836 87.88) (end 105.287 87.88) (width 0.13) (layer F.Cu) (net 7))
 (segment (start 100.838 87.376) (end 101.997 87.376) (width 0.13) (layer F.Cu) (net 7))
 (via (at 100.838 87.376) (size 0.4) (drill 0.25) (layers F.Cu B.Cu) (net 7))
 (segment (start 104.775 87.376) (end 100.838 87.376) (width 0.13) (layer B.Cu) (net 7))
 (segment (start 105.283 87.884) (end 104.775 87.376) (width 0.13) (layer B.Cu) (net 7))
 (via (at 105.283 87.884) (size 0.4) (drill 0.25) (layers F.Cu B.Cu) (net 7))
 (segment (start 105.287 87.88) (end 105.283 87.884) (width 0.13) (layer F.Cu) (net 7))
 (segment (start 106.836 87.38) (end 104.001 87.38) (width 0.13) (layer F.Cu) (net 8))
 (segment (start 104.001 87.38) (end 103.997 87.376) (width 0.13) (layer F.Cu) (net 8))
 (segment (start 106.836 85.88) (end 105.819 85.88) (width 0.13) (layer F.Cu) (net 9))
 (segment (start 100.838 81.788) (end 101.997 81.788) (width 0.13) (layer F.Cu) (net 9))
 (via (at 100.838 81.788) (size 0.4) (drill 0.25) (layers F.Cu B.Cu) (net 9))
 (segment (start 101.727 81.788) (end 100.838 81.788) (width 0.13) (layer B.Cu) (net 9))
 (segment (start 105.791 85.852) (end 101.727 81.788) (width 0.13) (layer B.Cu) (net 9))
 (via (at 105.791 85.852) (size 0.4) (drill 0.25) (layers F.Cu B.Cu) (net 9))
 (segment (start 105.819 85.88) (end 105.791 85.852) (width 0.13) (layer F.Cu) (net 9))
 (segment (start 106.836 85.38) (end 105.446 85.38) (width 0.13) (layer F.Cu) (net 10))
 (segment (start 105.41 83.201) (end 103.997 81.788) (width 0.13) (layer F.Cu) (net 10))
 (segment (start 105.41 85.344) (end 105.41 83.201) (width 0.13) (layer F.Cu) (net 10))
 (segment (start 105.446 85.38) (end 105.41 85.344) (width 0.13) (layer F.Cu) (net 10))
 (segment (start 106.836 88.88) (end 105.303 88.88) (width 0.13) (layer F.Cu) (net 30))
 (segment (start 104.902 90.485) (end 104.201 91.186) (width 0.13) (layer F.Cu) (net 30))
 (segment (start 104.902 89.281) (end 104.902 90.485) (width 0.13) (layer F.Cu) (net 30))
 (segment (start 105.303 88.88) (end 104.902 89.281) (width 0.13) (layer F.Cu) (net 30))
 (segment (start 105.029 94.168) (end 104.201 94.996) (width 0.13) (layer F.Cu) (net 31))
 (segment (start 105.029 92.837) (end 105.029 94.168) (width 0.13) (layer F.Cu) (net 31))
 (segment (start 105.664 92.202) (end 105.029 92.837) (width 0.13) (layer F.Cu) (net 31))
 (segment (start 105.664 90.551) (end 105.664 92.202) (width 0.13) (layer F.Cu) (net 31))
 (segment (start 105.835 90.38) (end 105.664 90.551) (width 0.13) (layer F.Cu) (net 31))
 (segment (start 106.836 90.38) (end 105.835 90.38) (width 0.13) (layer F.Cu) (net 31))
 (segment (start 106.836 86.88) (end 104.914 86.88) (width 0.13) (layer F.Cu) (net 32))
 (segment (start 104.902 86.172) (end 104.201 85.471) (width 0.13) (layer F.Cu) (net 32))
 (segment (start 104.902 86.868) (end 104.902 86.172) (width 0.13) (layer F.Cu) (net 32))
 (segment (start 104.914 86.88) (end 104.902 86.868) (width 0.13) (layer F.Cu) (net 32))
 (segment (start 106.836 88.38) (end 105.102 88.38) (width 0.13) (layer F.Cu) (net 33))
 (segment (start 105.102 88.38) (end 104.201 89.281) (width 0.13) (layer F.Cu) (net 33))
 (segment (start 106.836 84.88) (end 106.089 84.88) (width 0.13) (layer F.Cu) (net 34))
 (segment (start 105.156 80.8888) (end 104.1756 79.9084) (width 0.13) (layer F.Cu) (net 34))
 (segment (start 105.156 82.169) (end 105.156 80.8888) (width 0.13) (layer F.Cu) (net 34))
 (segment (start 105.791 82.804) (end 105.156 82.169) (width 0.13) (layer F.Cu) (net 34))
 (segment (start 105.791 84.582) (end 105.791 82.804) (width 0.13) (layer F.Cu) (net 34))
 (segment (start 106.089 84.88) (end 105.791 84.582) (width 0.13) (layer F.Cu) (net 34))
 (segment (start 106.836 86.38) (end 105.557 86.38) (width 0.13) (layer F.Cu) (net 35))
 (segment (start 105.029 84.455) (end 104.201 83.627) (width 0.13) (layer F.Cu) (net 35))
 (segment (start 105.029 85.725) (end 105.029 84.455) (width 0.13) (layer F.Cu) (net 35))
 (segment (start 105.283 85.979) (end 105.029 85.725) (width 0.13) (layer F.Cu) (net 35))
 (segment (start 105.283 86.106) (end 105.283 85.979) (width 0.13) (layer F.Cu) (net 35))
 (segment (start 105.557 86.38) (end 105.283 86.106) (width 0.13) (layer F.Cu) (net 35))
 (segment (start 104.201 83.627) (end 104.201 83.566) (width 0.13) (layer F.Cu) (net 35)))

